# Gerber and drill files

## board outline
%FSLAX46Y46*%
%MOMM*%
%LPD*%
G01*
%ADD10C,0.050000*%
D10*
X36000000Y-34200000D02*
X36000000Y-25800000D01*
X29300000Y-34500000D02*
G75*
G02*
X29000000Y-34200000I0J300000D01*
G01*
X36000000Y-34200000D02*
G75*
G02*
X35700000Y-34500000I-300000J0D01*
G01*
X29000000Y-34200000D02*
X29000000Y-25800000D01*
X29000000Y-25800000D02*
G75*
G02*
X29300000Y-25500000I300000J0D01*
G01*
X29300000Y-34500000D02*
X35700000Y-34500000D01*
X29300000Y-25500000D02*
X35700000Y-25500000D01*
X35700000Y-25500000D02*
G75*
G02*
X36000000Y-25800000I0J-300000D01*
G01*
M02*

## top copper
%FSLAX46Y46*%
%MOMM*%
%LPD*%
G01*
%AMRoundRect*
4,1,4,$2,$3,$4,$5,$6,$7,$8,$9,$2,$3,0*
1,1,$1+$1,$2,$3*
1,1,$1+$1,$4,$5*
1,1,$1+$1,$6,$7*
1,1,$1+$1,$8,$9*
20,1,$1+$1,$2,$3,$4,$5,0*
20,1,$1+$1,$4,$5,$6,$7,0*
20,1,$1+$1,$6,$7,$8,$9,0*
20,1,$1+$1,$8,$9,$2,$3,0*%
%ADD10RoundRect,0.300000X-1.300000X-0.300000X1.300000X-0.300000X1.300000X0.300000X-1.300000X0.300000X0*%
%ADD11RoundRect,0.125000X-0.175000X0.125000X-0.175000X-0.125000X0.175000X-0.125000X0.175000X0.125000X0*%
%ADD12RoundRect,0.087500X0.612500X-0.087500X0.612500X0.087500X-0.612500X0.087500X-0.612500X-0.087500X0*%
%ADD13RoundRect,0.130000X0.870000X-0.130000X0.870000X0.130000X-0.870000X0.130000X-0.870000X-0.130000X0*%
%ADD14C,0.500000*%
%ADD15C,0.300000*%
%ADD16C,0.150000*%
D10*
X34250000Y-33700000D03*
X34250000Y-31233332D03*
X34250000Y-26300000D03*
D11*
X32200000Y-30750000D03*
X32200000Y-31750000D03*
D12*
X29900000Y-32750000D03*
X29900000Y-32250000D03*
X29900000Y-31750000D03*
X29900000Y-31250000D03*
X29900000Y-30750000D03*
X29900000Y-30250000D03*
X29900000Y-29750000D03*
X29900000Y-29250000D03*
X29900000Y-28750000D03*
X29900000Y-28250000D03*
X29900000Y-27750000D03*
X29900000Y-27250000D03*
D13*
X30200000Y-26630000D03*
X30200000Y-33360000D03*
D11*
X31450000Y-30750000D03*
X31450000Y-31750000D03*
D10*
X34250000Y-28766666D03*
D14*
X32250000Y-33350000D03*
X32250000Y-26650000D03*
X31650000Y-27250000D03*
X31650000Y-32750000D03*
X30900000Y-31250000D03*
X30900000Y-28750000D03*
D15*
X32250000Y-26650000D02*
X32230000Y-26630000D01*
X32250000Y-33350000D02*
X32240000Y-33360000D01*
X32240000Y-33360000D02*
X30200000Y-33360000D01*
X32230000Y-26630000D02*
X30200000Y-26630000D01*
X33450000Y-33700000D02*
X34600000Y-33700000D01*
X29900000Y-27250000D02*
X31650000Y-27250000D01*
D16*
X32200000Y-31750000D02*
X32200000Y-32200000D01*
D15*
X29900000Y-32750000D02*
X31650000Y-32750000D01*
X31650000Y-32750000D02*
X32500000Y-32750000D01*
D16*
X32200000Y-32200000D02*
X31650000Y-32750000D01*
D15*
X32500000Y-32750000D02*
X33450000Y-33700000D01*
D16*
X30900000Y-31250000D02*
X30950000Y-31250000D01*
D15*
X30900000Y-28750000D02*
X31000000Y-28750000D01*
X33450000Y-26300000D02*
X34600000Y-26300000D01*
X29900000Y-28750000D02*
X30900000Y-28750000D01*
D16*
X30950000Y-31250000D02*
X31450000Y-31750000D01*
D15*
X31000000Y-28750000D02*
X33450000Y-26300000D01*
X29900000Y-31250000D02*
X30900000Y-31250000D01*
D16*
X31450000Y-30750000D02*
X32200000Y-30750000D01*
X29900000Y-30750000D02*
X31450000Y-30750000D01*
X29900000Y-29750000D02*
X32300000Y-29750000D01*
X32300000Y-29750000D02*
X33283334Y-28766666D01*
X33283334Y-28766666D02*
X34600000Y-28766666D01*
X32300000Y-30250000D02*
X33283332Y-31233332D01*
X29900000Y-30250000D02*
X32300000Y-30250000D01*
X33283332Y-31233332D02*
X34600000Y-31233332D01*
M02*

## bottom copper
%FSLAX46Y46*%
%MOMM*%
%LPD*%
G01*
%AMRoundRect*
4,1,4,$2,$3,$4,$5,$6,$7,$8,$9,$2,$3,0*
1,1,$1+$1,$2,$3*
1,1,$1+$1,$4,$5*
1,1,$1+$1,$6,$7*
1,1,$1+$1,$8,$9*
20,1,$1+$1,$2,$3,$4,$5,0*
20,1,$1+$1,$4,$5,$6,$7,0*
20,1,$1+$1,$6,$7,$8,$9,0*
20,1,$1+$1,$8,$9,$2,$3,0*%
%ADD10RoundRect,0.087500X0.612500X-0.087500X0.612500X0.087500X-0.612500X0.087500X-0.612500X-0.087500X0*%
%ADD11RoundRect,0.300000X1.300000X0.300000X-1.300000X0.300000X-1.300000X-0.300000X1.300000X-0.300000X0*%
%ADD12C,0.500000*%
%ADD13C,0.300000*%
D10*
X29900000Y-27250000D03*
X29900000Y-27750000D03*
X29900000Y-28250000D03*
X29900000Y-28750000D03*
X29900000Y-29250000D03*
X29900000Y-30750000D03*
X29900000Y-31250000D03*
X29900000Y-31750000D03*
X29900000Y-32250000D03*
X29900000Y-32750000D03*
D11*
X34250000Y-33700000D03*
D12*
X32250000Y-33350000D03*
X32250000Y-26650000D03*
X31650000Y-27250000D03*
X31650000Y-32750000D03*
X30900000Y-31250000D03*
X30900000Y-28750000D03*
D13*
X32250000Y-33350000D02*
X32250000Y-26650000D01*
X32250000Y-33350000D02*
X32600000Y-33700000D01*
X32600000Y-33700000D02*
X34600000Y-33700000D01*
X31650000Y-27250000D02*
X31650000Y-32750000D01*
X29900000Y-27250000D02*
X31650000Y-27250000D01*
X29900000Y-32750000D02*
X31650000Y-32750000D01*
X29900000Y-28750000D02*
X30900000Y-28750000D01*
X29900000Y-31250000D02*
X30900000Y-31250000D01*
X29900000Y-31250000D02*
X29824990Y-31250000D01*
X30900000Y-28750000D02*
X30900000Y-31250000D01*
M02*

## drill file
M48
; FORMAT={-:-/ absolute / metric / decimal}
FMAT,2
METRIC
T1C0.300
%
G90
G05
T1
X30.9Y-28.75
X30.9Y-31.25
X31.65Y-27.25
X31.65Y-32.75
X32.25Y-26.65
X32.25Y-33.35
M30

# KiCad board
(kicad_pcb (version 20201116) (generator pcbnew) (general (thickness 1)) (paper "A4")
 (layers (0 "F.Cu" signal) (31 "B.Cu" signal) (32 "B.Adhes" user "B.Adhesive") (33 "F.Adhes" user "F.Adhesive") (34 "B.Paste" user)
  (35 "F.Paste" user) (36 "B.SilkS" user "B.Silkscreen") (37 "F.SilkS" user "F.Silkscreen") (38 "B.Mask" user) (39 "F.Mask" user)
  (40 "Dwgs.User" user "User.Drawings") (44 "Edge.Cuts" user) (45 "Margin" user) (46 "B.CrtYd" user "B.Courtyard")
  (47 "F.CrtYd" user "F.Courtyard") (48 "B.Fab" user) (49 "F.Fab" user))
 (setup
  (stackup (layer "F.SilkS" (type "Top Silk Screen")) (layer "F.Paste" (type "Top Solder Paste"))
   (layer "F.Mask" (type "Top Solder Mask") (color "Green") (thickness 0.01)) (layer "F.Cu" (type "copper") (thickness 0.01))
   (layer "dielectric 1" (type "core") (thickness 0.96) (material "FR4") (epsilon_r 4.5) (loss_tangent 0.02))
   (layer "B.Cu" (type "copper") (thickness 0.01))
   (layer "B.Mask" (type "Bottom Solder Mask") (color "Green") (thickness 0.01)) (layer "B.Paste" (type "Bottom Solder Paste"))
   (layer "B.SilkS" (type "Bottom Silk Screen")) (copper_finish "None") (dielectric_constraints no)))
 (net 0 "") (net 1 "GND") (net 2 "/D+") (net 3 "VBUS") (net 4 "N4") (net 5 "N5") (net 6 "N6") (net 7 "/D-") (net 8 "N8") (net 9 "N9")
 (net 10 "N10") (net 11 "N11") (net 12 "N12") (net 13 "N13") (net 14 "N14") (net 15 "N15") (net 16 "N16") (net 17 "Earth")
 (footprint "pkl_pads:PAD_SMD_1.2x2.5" (layer "F.Cu") (at 34.6 33.7)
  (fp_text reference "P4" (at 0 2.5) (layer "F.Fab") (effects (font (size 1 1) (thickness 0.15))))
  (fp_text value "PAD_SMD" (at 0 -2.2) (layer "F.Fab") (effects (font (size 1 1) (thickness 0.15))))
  (pad "1" smd roundrect (at -0.35 0) (size 3.2 1.2) (layers "F.Cu" "F.Mask") (roundrect_rratio 0.25) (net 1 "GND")))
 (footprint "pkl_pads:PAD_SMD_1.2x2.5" (layer "F.Cu") (at 34.6 31.233332)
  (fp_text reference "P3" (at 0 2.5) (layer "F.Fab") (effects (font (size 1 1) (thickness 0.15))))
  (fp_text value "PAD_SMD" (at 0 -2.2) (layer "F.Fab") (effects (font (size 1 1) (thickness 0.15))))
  (pad "1" smd roundrect (at -0.35 0) (size 3.2 1.2) (layers "F.Cu" "F.Mask") (roundrect_rratio 0.25) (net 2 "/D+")))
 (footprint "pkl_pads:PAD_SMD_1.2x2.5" (layer "F.Cu") (at 34.6 26.3)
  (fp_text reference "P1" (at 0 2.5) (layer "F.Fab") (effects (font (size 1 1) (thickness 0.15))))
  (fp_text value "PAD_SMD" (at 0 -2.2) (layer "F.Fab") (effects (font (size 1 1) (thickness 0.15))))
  (pad "1" smd roundrect (at -0.35 0) (size 3.2 1.2) (layers "F.Cu" "F.Mask") (roundrect_rratio 0.25) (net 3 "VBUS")))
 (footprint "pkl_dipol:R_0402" (layer "F.Cu") (at 32.2 31.25 -90)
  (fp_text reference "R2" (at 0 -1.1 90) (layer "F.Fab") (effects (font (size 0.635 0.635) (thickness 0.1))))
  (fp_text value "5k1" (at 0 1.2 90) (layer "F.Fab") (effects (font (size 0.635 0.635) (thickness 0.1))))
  (pad "1" smd roundrect (at -0.5 0 270) (size 0.5 0.6) (layers "F.Cu" "F.Paste" "F.Mask") (roundrect_rratio 0.25) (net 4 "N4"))
  (pad "2" smd roundrect (at 0.5 0 270) (size 0.5 0.6) (layers "F.Cu" "F.Paste" "F.Mask") (roundrect_rratio 0.25) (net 1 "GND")))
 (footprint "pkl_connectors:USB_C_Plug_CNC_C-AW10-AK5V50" (layer "F.Cu") (at 30 30 90)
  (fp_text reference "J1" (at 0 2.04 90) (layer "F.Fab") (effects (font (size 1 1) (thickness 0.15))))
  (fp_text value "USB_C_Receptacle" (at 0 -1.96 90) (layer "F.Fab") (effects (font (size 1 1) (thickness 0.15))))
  (pad "A1" smd roundrect (at -2.75 -0.1 90) (size 0.35 1.4) (layers "F.Cu" "F.Paste" "F.Mask") (roundrect_rratio 0.25) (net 1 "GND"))
  (pad "A2" smd roundrect (at -2.25 -0.1 90) (size 0.35 1.4) (layers "F.Cu" "F.Paste" "F.Mask") (roundrect_rratio 0.25) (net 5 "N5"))
  (pad "A3" smd roundrect (at -1.75 -0.1 90) (size 0.35 1.4) (layers "F.Cu" "F.Paste" "F.Mask") (roundrect_rratio 0.25) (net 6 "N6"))
  (pad "A4" smd roundrect (at -1.25 -0.1 90) (size 0.35 1.4) (layers "F.Cu" "F.Paste" "F.Mask") (roundrect_rratio 0.25) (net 3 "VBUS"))
  (pad "A5" smd roundrect (at -0.75 -0.1 90) (size 0.35 1.4) (layers "F.Cu" "F.Paste" "F.Mask") (roundrect_rratio 0.25) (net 4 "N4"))
  (pad "A6" smd roundrect (at -0.25 -0.1 90) (size 0.35 1.4) (layers "F.Cu" "F.Paste" "F.Mask") (roundrect_rratio 0.25) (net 2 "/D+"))
  (pad "A7" smd roundrect (at 0.25 -0.1 90) (size 0.35 1.4) (layers "F.Cu" "F.Paste" "F.Mask") (roundrect_rratio 0.25) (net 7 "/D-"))
  (pad "A8" smd roundrect (at 0.75 -0.1 90) (size 0.35 1.4) (layers "F.Cu" "F.Paste" "F.Mask") (roundrect_rratio 0.25) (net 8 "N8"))
  (pad "A9" smd roundrect (at 1.25 -0.1 90) (size 0.35 1.4) (layers "F.Cu" "F.Paste" "F.Mask") (roundrect_rratio 0.25) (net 3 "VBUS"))
  (pad "A10" smd roundrect (at 1.75 -0.1 90) (size 0.35 1.4) (layers "F.Cu" "F.Paste" "F.Mask") (roundrect_rratio 0.25) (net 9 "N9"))
  (pad "A11" smd roundrect (at 2.25 -0.1 90) (size 0.35 1.4) (layers "F.Cu" "F.Paste" "F.Mask") (roundrect_rratio 0.25) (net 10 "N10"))
  (pad "A12" smd roundrect (at 2.75 -0.1 90) (size 0.35 1.4) (layers "F.Cu" "F.Paste" "F.Mask") (roundrect_rratio 0.25) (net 1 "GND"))
  (pad "B1" smd roundrect (at 2.75 -0.1 90) (size 0.35 1.4) (layers "B.Cu" "B.Paste" "B.Mask") (roundrect_rratio 0.25) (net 1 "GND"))
  (pad "B2" smd roundrect (at 2.25 -0.1 90) (size 0.35 1.4) (layers "B.Cu" "B.Paste" "B.Mask") (roundrect_rratio 0.25) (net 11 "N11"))
  (pad "B3" smd roundrect (at 1.75 -0.1 90) (size 0.35 1.4) (layers "B.Cu" "B.Paste" "B.Mask") (roundrect_rratio 0.25) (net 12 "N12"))
  (pad "B4" smd roundrect (at 1.25 -0.1 90) (size 0.35 1.4) (layers "B.Cu" "B.Paste" "B.Mask") (roundrect_rratio 0.25) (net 3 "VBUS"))
  (pad "B5" smd roundrect (at 0.75 -0.1 90) (size 0.35 1.4) (layers "B.Cu" "B.Paste" "B.Mask") (roundrect_rratio 0.25) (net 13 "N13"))
  (pad "B8" smd roundrect (at -0.75 -0.1 90) (size 0.35 1.4) (layers "B.Cu" "B.Paste" "B.Mask") (roundrect_rratio 0.25) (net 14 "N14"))
  (pad "B9" smd roundrect (at -1.25 -0.1 90) (size 0.35 1.4) (layers "B.Cu" "B.Paste" "B.Mask") (roundrect_rratio 0.25) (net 3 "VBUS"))
  (pad "B10" smd roundrect (at -1.75 -0.1 90) (size 0.35 1.4) (layers "B.Cu" "B.Paste" "B.Mask") (roundrect_rratio 0.25) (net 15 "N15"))
  (pad "B11" smd roundrect (at -2.25 -0.1 90) (size 0.35 1.4) (layers "B.Cu" "B.Paste" "B.Mask") (roundrect_rratio 0.25) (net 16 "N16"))
  (pad "B12" smd roundrect (at -2.75 -0.1 90) (size 0.35 1.4) (layers "B.Cu" "B.Paste" "B.Mask") (roundrect_rratio 0.25) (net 1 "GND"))
  (pad "S1" smd roundrect (at 3.37 0.2 90) (size 0.52 2) (layers "F.Cu" "F.Paste" "F.Mask") (roundrect_rratio 0.25) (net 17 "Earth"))
  (pad "S1" smd roundrect (at -3.36 0.2 90) (size 0.52 2) (layers "F.Cu" "F.Paste" "F.Mask") (roundrect_rratio 0.25) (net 17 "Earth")))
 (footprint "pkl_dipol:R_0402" (layer "F.Cu") (at 31.45 31.25 -90)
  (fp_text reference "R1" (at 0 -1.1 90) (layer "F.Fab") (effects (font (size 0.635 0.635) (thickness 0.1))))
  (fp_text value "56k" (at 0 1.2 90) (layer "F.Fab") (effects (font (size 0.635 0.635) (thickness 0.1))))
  (pad "1" smd roundrect (at -0.5 0 270) (size 0.5 0.6) (layers "F.Cu" "F.Paste" "F.Mask") (roundrect_rratio 0.25) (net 4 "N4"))
  (pad "2" smd roundrect (at 0.5 0 270) (size 0.5 0.6) (layers "F.Cu" "F.Paste" "F.Mask") (roundrect_rratio 0.25) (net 3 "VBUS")))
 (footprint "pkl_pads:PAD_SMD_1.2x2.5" (layer "F.Cu") (at 34.6 28.766666)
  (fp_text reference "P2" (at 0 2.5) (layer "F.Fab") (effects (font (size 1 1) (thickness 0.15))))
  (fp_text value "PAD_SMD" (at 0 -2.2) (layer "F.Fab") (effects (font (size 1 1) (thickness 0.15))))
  (pad "1" smd roundrect (at -0.35 0) (size 3.2 1.2) (layers "F.Cu" "F.Mask") (roundrect_rratio 0.25) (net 7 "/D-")))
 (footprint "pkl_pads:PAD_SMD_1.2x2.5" (layer "B.Cu") (at 34.6 33.7 180)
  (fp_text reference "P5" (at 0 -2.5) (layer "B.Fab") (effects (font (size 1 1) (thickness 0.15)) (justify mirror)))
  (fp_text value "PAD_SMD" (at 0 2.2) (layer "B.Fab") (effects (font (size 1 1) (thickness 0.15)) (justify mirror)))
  (pad "1" smd roundrect (at 0.35 0 180) (size 3.2 1.2) (layers "B.Cu" "B.Mask") (roundrect_rratio 0.25) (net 17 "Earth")))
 (gr_line (start 36 34.2) (end 36 25.8) (layer "Edge.Cuts") (width 0.05))
 (gr_arc (start 29.3 34.2) (end 29 34.2) (angle -90) (layer "Edge.Cuts") (width 0.05))
 (gr_arc (start 35.7 34.2) (end 35.7 34.5) (angle -90) (layer "Edge.Cuts") (width 0.05))
 (gr_line (start 29 34.2) (end 29 25.8) (layer "Edge.Cuts") (width 0.05))
 (gr_arc (start 29.3 25.8) (end 29 25.8) (angle 90) (layer "Edge.Cuts") (width 0.05))
 (gr_line (start 29.3 34.5) (end 35.7 34.5) (layer "Edge.Cuts") (width 0.05))
 (gr_line (start 29.3 25.5) (end 35.7 25.5) (layer "Edge.Cuts") (width 0.05))
 (gr_arc (start 35.7 25.8) (end 36 25.8) (angle -90) (layer "Edge.Cuts") (width 0.05))
 (segment (start 32.25 26.65) (end 32.23 26.63) (width 0.3) (layer "F.Cu") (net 17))
 (segment (start 32.25 33.35) (end 32.24 33.36) (width 0.3) (layer "F.Cu") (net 17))
 (segment (start 32.24 33.36) (end 30.2 33.36) (width 0.3) (layer "F.Cu") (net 17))
 (segment (start 32.23 26.63) (end 30.2 26.63) (width 0.3) (layer "F.Cu") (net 17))
 (via (at 32.25 33.35) (size 0.5) (drill 0.3) (layers "F.Cu" "B.Cu") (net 17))
 (via (at 32.25 26.65) (size 0.5) (drill 0.3) (layers "F.Cu" "B.Cu") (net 17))
 (segment (start 32.25 33.35) (end 32.25 26.65) (width 0.3) (layer "B.Cu") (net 17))
 (segment (start 32.25 33.35) (end 32.6 33.7) (width 0.3) (layer "B.Cu") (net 17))
 (segment (start 32.6 33.7) (end 34.6 33.7) (width 0.3) (layer "B.Cu") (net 17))
 (segment (start 33.45 33.7) (end 34.6 33.7) (width 0.3) (layer "F.Cu") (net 1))
 (segment (start 29.9 27.25) (end 31.65 27.25) (width 0.3) (layer "F.Cu") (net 1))
 (segment (start 32.2 31.75) (end 32.2 32.2) (width 0.15) (layer "F.Cu") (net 1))
 (segment (start 29.9 32.75) (end 31.65 32.75) (width 0.3) (layer "F.Cu") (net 1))
 (segment (start 31.65 32.75) (end 32.5 32.75) (width 0.3) (layer "F.Cu") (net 1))
 (segment (start 32.2 32.2) (end 31.65 32.75) (width 0.15) (layer "F.Cu") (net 1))
 (segment (start 32.5 32.75) (end 33.45 33.7) (width 0.3) (layer "F.Cu") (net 1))
 (via (at 31.65 27.25) (size 0.5) (drill 0.3) (layers "F.Cu" "B.Cu") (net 1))
 (via (at 31.65 32.75) (size 0.5) (drill 0.3) (layers "F.Cu" "B.Cu") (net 1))
 (segment (start 31.65 27.25) (end 31.65 32.75) (width 0.3) (layer "B.Cu") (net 1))
 (segment (start 29.9 27.25) (end 31.65 27.25) (width 0.3) (layer "B.Cu") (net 1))
 (segment (start 29.9 32.75) (end 31.65 32.75) (width 0.3) (layer "B.Cu") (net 1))
 (segment (start 30.9 31.25) (end 30.95 31.25) (width 0.15) (layer "F.Cu") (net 3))
 (segment (start 30.9 28.75) (end 31 28.75) (width 0.3) (layer "F.Cu") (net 3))
 (segment (start 33.45 26.3) (end 34.6 26.3) (width 0.3) (layer "F.Cu") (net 3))
 (segment (start 29.9 28.75) (end 30.9 28.75) (width 0.3) (layer "F.Cu") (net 3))
 (segment (start 30.95 31.25) (end 31.45 31.75) (width 0.15) (layer "F.Cu") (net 3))
 (segment (start 31 28.75) (end 33.45 26.3) (width 0.3) (layer "F.Cu") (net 3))
 (segment (start 29.9 31.25) (end 30.9 31.25) (width 0.3) (layer "F.Cu") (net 3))
 (via (at 30.9 31.25) (size 0.5) (drill 0.3) (layers "F.Cu" "B.Cu") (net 3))
 (via (at 30.9 28.75) (size 0.5) (drill 0.3) (layers "F.Cu" "B.Cu") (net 3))
 (segment (start 29.9 28.75) (end 30.9 28.75) (width 0.3) (layer "B.Cu") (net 3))
 (segment (start 29.9 31.25) (end 30.9 31.25) (width 0.3) (layer "B.Cu") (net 3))
 (segment (start 29.9 31.25) (end 29.82499 31.25) (width 0.3) (layer "B.Cu") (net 3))
 (segment (start 30.9 28.75) (end 30.9 31.25) (width 0.3) (layer "B.Cu") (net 3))
 (segment (start 31.45 30.75) (end 32.2 30.75) (width 0.15) (layer "F.Cu") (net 4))
 (segment (start 29.9 30.75) (end 31.45 30.75) (width 0.15) (layer "F.Cu") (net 4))
 (segment (start 29.9 29.75) (end 32.3 29.75) (width 0.15) (layer "F.Cu") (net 7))
 (segment (start 32.3 29.75) (end 33.283334 28.766666) (width 0.15) (layer "F.Cu") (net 7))
 (segment (start 33.283334 28.766666) (end 34.6 28.766666) (width 0.15) (layer "F.Cu") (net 7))
 (segment (start 32.3 30.25) (end 33.283332 31.233332) (width 0.15) (layer "F.Cu") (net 2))
 (segment (start 29.9 30.25) (end 32.3 30.25) (width 0.15) (layer "F.Cu") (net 2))
 (segment (start 33.283332 31.233332) (end 34.6 31.233332) (width 0.15) (layer "F.Cu") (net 2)))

